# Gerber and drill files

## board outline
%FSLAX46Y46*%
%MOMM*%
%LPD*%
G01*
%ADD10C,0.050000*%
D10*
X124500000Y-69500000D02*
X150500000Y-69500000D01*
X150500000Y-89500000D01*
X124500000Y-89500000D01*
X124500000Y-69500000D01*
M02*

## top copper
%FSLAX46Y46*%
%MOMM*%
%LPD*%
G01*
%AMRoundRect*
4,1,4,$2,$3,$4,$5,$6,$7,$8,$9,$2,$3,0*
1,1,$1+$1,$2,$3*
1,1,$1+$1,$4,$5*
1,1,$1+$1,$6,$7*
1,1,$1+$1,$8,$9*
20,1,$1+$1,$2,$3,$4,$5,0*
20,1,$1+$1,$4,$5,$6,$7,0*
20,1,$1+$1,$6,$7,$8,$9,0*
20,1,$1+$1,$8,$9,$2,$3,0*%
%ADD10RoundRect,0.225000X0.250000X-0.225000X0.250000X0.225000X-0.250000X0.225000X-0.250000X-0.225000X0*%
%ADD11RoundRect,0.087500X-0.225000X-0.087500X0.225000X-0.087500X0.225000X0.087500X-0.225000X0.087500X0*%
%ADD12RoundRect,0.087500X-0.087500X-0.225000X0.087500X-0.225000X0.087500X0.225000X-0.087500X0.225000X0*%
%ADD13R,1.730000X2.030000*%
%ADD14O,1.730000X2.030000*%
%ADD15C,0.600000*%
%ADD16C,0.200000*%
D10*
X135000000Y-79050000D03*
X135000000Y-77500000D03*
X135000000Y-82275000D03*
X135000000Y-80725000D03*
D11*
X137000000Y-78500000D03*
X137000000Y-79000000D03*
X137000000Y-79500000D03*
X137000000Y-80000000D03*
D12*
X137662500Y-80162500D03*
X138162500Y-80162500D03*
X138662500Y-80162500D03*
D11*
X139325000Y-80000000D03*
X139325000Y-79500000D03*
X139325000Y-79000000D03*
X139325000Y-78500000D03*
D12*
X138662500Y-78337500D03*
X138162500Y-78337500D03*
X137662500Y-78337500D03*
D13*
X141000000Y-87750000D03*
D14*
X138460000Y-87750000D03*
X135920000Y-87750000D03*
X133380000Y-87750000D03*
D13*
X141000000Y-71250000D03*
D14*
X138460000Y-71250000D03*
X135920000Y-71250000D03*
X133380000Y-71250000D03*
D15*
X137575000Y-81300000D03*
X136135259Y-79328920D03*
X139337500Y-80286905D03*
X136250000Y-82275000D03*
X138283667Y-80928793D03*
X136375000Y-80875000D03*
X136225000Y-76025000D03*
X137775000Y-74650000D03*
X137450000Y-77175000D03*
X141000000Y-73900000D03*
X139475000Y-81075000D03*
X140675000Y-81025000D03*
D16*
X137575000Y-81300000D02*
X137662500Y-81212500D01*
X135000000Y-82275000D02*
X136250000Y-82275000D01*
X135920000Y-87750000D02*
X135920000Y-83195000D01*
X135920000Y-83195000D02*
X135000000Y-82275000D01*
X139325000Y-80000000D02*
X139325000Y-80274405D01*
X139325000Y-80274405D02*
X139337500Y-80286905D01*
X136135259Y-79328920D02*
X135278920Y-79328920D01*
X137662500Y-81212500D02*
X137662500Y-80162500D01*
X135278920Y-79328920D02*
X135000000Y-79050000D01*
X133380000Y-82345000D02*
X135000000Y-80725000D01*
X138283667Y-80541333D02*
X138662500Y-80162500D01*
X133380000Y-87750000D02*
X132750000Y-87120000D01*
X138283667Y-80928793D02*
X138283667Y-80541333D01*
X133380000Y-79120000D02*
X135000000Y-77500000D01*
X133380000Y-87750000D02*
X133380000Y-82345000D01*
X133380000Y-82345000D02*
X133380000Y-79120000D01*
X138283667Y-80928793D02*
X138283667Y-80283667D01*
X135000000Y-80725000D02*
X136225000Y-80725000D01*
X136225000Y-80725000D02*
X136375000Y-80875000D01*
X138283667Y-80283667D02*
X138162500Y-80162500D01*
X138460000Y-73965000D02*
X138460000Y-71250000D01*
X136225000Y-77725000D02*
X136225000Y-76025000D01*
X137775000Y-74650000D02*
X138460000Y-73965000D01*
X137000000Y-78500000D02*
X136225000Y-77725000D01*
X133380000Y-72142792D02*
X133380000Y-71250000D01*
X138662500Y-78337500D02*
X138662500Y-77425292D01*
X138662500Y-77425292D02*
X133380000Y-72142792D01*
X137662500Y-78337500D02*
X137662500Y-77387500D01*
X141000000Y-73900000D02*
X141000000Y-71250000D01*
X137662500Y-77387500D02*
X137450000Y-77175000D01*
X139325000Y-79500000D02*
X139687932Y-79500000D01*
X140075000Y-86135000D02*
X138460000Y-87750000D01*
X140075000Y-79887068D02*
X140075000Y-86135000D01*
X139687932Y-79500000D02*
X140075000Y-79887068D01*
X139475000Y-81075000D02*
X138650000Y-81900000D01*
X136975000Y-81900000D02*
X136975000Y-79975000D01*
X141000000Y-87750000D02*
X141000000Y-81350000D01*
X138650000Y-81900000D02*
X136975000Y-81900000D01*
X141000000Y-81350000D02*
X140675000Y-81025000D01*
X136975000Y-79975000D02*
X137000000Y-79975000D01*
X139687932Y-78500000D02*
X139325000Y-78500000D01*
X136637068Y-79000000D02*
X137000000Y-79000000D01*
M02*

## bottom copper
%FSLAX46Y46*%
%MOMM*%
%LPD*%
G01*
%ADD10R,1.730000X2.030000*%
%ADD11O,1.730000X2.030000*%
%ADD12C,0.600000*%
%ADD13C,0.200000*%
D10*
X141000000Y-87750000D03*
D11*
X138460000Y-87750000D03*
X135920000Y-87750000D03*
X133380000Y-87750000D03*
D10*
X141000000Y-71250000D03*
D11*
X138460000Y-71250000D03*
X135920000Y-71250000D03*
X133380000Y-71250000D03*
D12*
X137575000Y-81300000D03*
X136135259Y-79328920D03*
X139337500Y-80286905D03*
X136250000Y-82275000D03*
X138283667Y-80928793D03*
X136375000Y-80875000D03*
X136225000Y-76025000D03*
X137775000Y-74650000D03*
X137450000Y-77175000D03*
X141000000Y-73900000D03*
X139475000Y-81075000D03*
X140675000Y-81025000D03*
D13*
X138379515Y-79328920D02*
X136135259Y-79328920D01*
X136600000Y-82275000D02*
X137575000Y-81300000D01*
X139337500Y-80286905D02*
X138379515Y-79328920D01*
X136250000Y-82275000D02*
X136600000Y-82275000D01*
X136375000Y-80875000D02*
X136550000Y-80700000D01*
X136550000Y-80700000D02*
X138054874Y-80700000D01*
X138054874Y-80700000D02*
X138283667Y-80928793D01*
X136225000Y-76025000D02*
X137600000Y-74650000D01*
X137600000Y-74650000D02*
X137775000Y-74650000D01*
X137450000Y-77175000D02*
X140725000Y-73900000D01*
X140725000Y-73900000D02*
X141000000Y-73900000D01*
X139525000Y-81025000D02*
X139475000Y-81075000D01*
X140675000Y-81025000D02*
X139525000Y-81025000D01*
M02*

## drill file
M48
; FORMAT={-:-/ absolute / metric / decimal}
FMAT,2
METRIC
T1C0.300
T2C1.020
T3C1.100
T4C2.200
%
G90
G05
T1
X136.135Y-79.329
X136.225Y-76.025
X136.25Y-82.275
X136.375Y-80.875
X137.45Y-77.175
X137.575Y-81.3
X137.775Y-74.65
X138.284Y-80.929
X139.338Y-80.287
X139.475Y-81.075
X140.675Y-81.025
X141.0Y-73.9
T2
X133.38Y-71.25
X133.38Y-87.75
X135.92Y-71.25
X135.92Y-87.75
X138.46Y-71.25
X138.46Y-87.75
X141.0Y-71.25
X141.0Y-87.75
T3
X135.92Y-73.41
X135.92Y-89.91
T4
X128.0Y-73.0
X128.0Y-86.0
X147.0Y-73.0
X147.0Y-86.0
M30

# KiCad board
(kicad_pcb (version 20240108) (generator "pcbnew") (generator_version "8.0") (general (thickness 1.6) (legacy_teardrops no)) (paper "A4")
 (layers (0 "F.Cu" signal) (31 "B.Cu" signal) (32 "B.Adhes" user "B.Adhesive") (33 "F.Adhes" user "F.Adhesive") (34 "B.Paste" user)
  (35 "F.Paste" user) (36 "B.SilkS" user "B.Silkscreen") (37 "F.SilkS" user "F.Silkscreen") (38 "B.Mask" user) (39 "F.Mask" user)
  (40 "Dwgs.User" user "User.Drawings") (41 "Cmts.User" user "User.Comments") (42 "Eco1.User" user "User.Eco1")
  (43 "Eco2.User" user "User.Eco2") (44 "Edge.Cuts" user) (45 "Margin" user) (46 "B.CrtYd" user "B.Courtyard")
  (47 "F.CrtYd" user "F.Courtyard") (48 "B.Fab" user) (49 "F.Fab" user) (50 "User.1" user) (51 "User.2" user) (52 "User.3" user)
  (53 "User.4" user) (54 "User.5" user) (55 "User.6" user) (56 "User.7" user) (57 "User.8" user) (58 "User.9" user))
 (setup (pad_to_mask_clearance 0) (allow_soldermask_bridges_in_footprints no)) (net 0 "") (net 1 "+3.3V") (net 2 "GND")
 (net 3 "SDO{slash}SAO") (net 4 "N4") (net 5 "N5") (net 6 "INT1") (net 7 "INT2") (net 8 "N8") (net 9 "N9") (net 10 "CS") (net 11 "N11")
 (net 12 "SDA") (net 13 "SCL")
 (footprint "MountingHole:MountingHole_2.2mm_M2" (layer "F.Cu") (at 128 86)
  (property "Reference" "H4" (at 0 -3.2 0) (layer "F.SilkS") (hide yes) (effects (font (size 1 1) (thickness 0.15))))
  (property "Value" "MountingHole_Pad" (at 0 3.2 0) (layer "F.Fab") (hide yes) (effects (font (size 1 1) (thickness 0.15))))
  (pad "" np_thru_hole circle (at 0 0) (size 2.2 2.2) (drill 2.2) (layers "*.Cu" "*.Mask")))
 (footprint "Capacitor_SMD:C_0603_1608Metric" (layer "F.Cu") (at 135 78.275 90)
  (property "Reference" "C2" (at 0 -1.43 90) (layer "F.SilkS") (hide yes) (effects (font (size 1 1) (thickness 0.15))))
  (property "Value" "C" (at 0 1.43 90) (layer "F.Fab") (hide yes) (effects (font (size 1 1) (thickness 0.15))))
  (pad "1" smd roundrect (at -0.775 0 90) (size 0.9 0.95) (layers "F.Cu" "F.Paste" "F.Mask") (roundrect_rratio 0.25) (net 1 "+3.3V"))
  (pad "2" smd roundrect (at 0.775 0 90) (size 0.9 0.95) (layers "F.Cu" "F.Paste" "F.Mask") (roundrect_rratio 0.25) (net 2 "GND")))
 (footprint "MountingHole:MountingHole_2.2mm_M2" (layer "F.Cu") (at 147 86)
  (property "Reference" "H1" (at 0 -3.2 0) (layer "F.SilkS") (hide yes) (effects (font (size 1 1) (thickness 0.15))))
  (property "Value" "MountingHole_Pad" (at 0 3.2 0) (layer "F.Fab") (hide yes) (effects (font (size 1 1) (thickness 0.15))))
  (pad "" np_thru_hole circle (at 0 0) (size 2.2 2.2) (drill 2.2) (layers "*.Cu" "*.Mask")))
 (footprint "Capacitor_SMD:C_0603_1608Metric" (layer "F.Cu") (at 135 81.5 90)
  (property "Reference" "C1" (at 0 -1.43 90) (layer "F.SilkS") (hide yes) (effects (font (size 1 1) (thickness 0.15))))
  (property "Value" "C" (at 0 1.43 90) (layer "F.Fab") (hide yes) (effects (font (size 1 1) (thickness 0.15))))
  (pad "1" smd roundrect (at -0.775 0 90) (size 0.9 0.95) (layers "F.Cu" "F.Paste" "F.Mask") (roundrect_rratio 0.25) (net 1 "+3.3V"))
  (pad "2" smd roundrect (at 0.775 0 90) (size 0.9 0.95) (layers "F.Cu" "F.Paste" "F.Mask") (roundrect_rratio 0.25) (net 2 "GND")))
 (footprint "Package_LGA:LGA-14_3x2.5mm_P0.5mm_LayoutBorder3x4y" (layer "F.Cu") (at 138.1625 79.25)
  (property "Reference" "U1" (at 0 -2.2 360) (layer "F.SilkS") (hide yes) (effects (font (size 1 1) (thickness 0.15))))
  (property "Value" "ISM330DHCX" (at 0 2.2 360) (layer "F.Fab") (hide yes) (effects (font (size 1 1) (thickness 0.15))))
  (pad "1" smd roundrect (at -1.1625 -0.75) (size 0.625 0.35) (layers "F.Cu" "F.Paste" "F.Mask") (roundrect_rratio 0.25)
   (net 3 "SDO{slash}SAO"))
  (pad "2" smd roundrect (at -1.1625 -0.25) (size 0.625 0.35) (layers "F.Cu" "F.Paste" "F.Mask") (roundrect_rratio 0.25) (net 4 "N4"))
  (pad "3" smd roundrect (at -1.1625 0.25) (size 0.625 0.35) (layers "F.Cu" "F.Paste" "F.Mask") (roundrect_rratio 0.25) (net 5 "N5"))
  (pad "4" smd roundrect (at -1.1625 0.75) (size 0.625 0.35) (layers "F.Cu" "F.Paste" "F.Mask") (roundrect_rratio 0.25) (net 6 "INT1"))
  (pad "5" smd roundrect (at -0.5 0.9125) (size 0.35 0.625) (layers "F.Cu" "F.Paste" "F.Mask") (roundrect_rratio 0.25) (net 1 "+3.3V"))
  (pad "6" smd roundrect (at 0 0.9125) (size 0.35 0.625) (layers "F.Cu" "F.Paste" "F.Mask") (roundrect_rratio 0.25) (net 2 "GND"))
  (pad "7" smd roundrect (at 0.5 0.9125) (size 0.35 0.625) (layers "F.Cu" "F.Paste" "F.Mask") (roundrect_rratio 0.25) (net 2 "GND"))
  (pad "8" smd roundrect (at 1.1625 0.75) (size 0.625 0.35) (layers "F.Cu" "F.Paste" "F.Mask") (roundrect_rratio 0.25) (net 1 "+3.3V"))
  (pad "9" smd roundrect (at 1.1625 0.25) (size 0.625 0.35) (layers "F.Cu" "F.Paste" "F.Mask") (roundrect_rratio 0.25) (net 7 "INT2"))
  (pad "10" smd roundrect (at 1.1625 -0.25) (size 0.625 0.35) (layers "F.Cu" "F.Paste" "F.Mask") (roundrect_rratio 0.25) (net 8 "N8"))
  (pad "11" smd roundrect (at 1.1625 -0.75) (size 0.625 0.35) (layers "F.Cu" "F.Paste" "F.Mask") (roundrect_rratio 0.25) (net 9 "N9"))
  (pad "12" smd roundrect (at 0.5 -0.9125) (size 0.35 0.625) (layers "F.Cu" "F.Paste" "F.Mask") (roundrect_rratio 0.25) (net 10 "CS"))
  (pad "13" smd roundrect (at 0 -0.9125) (size 0.35 0.625) (layers "F.Cu" "F.Paste" "F.Mask") (roundrect_rratio 0.25) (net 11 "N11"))
  (pad "14" smd roundrect (at -0.5 -0.9125) (size 0.35 0.625) (layers "F.Cu" "F.Paste" "F.Mask") (roundrect_rratio 0.25) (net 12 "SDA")))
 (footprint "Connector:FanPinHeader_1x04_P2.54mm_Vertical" (layer "F.Cu") (at 141 87.75 180)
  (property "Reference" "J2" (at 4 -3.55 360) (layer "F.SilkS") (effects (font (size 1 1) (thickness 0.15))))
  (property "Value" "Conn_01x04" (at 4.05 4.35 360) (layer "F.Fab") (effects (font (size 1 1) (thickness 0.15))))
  (pad "" np_thru_hole circle (at 5.08 -2.16 270) (size 1.1 1.1) (drill 1.1) (layers "*.Cu" "*.Mask"))
  (pad "1" thru_hole rect (at 0 0 270) (size 2.03 1.73) (drill 1.02) (layers "*.Cu" "*.Mask") (remove_unused_layers no) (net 6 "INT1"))
  (pad "2" thru_hole oval (at 2.54 0 270) (size 2.03 1.73) (drill 1.02) (layers "*.Cu" "*.Mask") (remove_unused_layers no) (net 7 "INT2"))
  (pad "3" thru_hole oval (at 5.08 0 270) (size 2.03 1.73) (drill 1.02) (layers "*.Cu" "*.Mask") (remove_unused_layers no) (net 1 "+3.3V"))
  (pad "4" thru_hole oval (at 7.62 0 270) (size 2.03 1.73) (drill 1.02) (layers "*.Cu" "*.Mask") (remove_unused_layers no) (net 2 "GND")))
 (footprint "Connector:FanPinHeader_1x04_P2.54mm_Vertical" (layer "F.Cu") (at 141 71.25 180)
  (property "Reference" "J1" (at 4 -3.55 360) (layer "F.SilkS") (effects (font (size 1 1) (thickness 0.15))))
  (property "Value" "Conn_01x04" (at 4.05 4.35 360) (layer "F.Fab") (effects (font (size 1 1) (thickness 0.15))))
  (pad "" np_thru_hole circle (at 5.08 -2.16 270) (size 1.1 1.1) (drill 1.1) (layers "*.Cu" "*.Mask"))
  (pad "1" thru_hole rect (at 0 0 270) (size 2.03 1.73) (drill 1.02) (layers "*.Cu" "*.Mask") (remove_unused_layers no) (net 12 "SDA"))
  (pad "2" thru_hole oval (at 2.54 0 270) (size 2.03 1.73) (drill 1.02) (layers "*.Cu" "*.Mask") (remove_unused_layers no)
   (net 3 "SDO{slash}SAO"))
  (pad "3" thru_hole oval (at 5.08 0 270) (size 2.03 1.73) (drill 1.02) (layers "*.Cu" "*.Mask") (remove_unused_layers no) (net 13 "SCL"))
  (pad "4" thru_hole oval (at 7.62 0 270) (size 2.03 1.73) (drill 1.02) (layers "*.Cu" "*.Mask") (remove_unused_layers no) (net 10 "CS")))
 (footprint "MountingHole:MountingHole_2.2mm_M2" (layer "F.Cu") (at 147 73)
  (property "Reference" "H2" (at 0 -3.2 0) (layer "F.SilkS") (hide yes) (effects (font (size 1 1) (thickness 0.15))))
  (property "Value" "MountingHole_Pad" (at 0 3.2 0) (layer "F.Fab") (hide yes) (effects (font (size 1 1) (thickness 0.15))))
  (pad "" np_thru_hole circle (at 0 0) (size 2.2 2.2) (drill 2.2) (layers "*.Cu" "*.Mask")))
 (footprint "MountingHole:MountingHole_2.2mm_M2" (layer "F.Cu") (at 128 73)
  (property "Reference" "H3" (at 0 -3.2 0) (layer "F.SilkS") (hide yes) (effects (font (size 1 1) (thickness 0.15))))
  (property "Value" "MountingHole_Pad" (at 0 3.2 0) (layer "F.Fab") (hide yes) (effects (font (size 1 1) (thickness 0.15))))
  (pad "" np_thru_hole circle (at 0 0) (size 2.2 2.2) (drill 2.2) (layers "*.Cu" "*.Mask")))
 (gr_rect (start 124.5 69.5) (end 150.5 89.5) (stroke (width 0.05) (type default)) (fill none) (layer "Edge.Cuts"))
 (segment (start 137.575 81.3) (end 137.6625 81.2125) (width 0.2) (layer "F.Cu") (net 1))
 (segment (start 135 82.275) (end 136.25 82.275) (width 0.2) (layer "F.Cu") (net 1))
 (segment (start 135.92 87.75) (end 135.92 83.195) (width 0.2) (layer "F.Cu") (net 1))
 (segment (start 135.92 83.195) (end 135 82.275) (width 0.2) (layer "F.Cu") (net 1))
 (segment (start 139.325 80) (end 139.325 80.274405) (width 0.2) (layer "F.Cu") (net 1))
 (segment (start 139.325 80.274405) (end 139.3375 80.286905) (width 0.2) (layer "F.Cu") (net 1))
 (segment (start 136.135259 79.32892) (end 135.27892 79.32892) (width 0.2) (layer "F.Cu") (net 1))
 (segment (start 137.6625 81.2125) (end 137.6625 80.1625) (width 0.2) (layer "F.Cu") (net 1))
 (segment (start 135.27892 79.32892) (end 135 79.05) (width 0.2) (layer "F.Cu") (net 1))
 (via (at 137.575 81.3) (size 0.6) (drill 0.3) (layers "F.Cu" "B.Cu") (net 1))
 (via (at 136.135259 79.32892) (size 0.6) (drill 0.3) (layers "F.Cu" "B.Cu") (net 1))
 (via (at 139.3375 80.286905) (size 0.6) (drill 0.3) (layers "F.Cu" "B.Cu") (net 1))
 (via (at 136.25 82.275) (size 0.6) (drill 0.3) (layers "F.Cu" "B.Cu") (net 1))
 (segment (start 138.379515 79.32892) (end 136.135259 79.32892) (width 0.2) (layer "B.Cu") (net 1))
 (segment (start 136.6 82.275) (end 137.575 81.3) (width 0.2) (layer "B.Cu") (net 1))
 (segment (start 139.3375 80.286905) (end 138.379515 79.32892) (width 0.2) (layer "B.Cu") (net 1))
 (segment (start 136.25 82.275) (end 136.6 82.275) (width 0.2) (layer "B.Cu") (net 1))
 (segment (start 133.38 82.345) (end 135 80.725) (width 0.2) (layer "F.Cu") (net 2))
 (segment (start 138.283667 80.541333) (end 138.6625 80.1625) (width 0.2) (layer "F.Cu") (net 2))
 (segment (start 133.38 87.75) (end 132.75 87.12) (width 0.2) (layer "F.Cu") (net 2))
 (segment (start 138.283667 80.928793) (end 138.283667 80.541333) (width 0.2) (layer "F.Cu") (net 2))
 (segment (start 133.38 79.12) (end 135 77.5) (width 0.2) (layer "F.Cu") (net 2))
 (segment (start 133.38 87.75) (end 133.38 82.345) (width 0.2) (layer "F.Cu") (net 2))
 (segment (start 133.38 82.345) (end 133.38 79.12) (width 0.2) (layer "F.Cu") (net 2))
 (segment (start 138.283667 80.928793) (end 138.283667 80.283667) (width 0.2) (layer "F.Cu") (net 2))
 (segment (start 135 80.725) (end 136.225 80.725) (width 0.2) (layer "F.Cu") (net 2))
 (segment (start 136.225 80.725) (end 136.375 80.875) (width 0.2) (layer "F.Cu") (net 2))
 (segment (start 138.283667 80.283667) (end 138.1625 80.1625) (width 0.2) (layer "F.Cu") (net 2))
 (via (at 138.283667 80.928793) (size 0.6) (drill 0.3) (layers "F.Cu" "B.Cu") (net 2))
 (via (at 136.375 80.875) (size 0.6) (drill 0.3) (layers "F.Cu" "B.Cu") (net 2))
 (segment (start 136.375 80.875) (end 136.55 80.7) (width 0.2) (layer "B.Cu") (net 2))
 (segment (start 136.55 80.7) (end 138.054874 80.7) (width 0.2) (layer "B.Cu") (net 2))
 (segment (start 138.054874 80.7) (end 138.283667 80.928793) (width 0.2) (layer "B.Cu") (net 2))
 (segment (start 138.46 73.965) (end 138.46 71.25) (width 0.2) (layer "F.Cu") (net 3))
 (segment (start 136.225 77.725) (end 136.225 76.025) (width 0.2) (layer "F.Cu") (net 3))
 (segment (start 137.775 74.65) (end 138.46 73.965) (width 0.2) (layer "F.Cu") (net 3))
 (segment (start 137 78.5) (end 136.225 77.725) (width 0.2) (layer "F.Cu") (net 3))
 (via (at 136.225 76.025) (size 0.6) (drill 0.3) (layers "F.Cu" "B.Cu") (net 3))
 (via (at 137.775 74.65) (size 0.6) (drill 0.3) (layers "F.Cu" "B.Cu") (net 3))
 (segment (start 136.225 76.025) (end 137.6 74.65) (width 0.2) (layer "B.Cu") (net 3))
 (segment (start 137.6 74.65) (end 137.775 74.65) (width 0.2) (layer "B.Cu") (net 3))
 (segment (start 133.38 72.142792) (end 133.38 71.25) (width 0.2) (layer "F.Cu") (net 10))
 (segment (start 138.6625 78.3375) (end 138.6625 77.425292) (width 0.2) (layer "F.Cu") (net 10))
 (segment (start 138.6625 77.425292) (end 133.38 72.142792) (width 0.2) (layer "F.Cu") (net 10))
 (segment (start 137.6625 78.3375) (end 137.6625 77.3875) (width 0.2) (layer "F.Cu") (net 12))
 (segment (start 141 73.9) (end 141 71.25) (width 0.2) (layer "F.Cu") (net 12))
 (segment (start 137.6625 77.3875) (end 137.45 77.175) (width 0.2) (layer "F.Cu") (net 12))
 (via (at 137.45 77.175) (size 0.6) (drill 0.3) (layers "F.Cu" "B.Cu") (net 12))
 (via (at 141 73.9) (size 0.6) (drill 0.3) (layers "F.Cu" "B.Cu") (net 12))
 (segment (start 137.45 77.175) (end 140.725 73.9) (width 0.2) (layer "B.Cu") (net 12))
 (segment (start 140.725 73.9) (end 141 73.9) (width 0.2) (layer "B.Cu") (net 12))
 (segment (start 139.325 79.5) (end 139.687932 79.5) (width 0.2) (layer "F.Cu") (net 7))
 (segment (start 140.075 86.135) (end 138.46 87.75) (width 0.2) (layer "F.Cu") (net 7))
 (segment (start 140.075 79.887068) (end 140.075 86.135) (width 0.2) (layer "F.Cu") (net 7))
 (segment (start 139.687932 79.5) (end 140.075 79.887068) (width 0.2) (layer "F.Cu") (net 7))
 (segment (start 139.475 81.075) (end 138.65 81.9) (width 0.2) (layer "F.Cu") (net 6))
 (segment (start 136.975 81.9) (end 136.975 79.975) (width 0.2) (layer "F.Cu") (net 6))
 (segment (start 141 87.75) (end 141 81.35) (width 0.2) (layer "F.Cu") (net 6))
 (segment (start 138.65 81.9) (end 136.975 81.9) (width 0.2) (layer "F.Cu") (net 6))
 (segment (start 141 81.35) (end 140.675 81.025) (width 0.2) (layer "F.Cu") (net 6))
 (segment (start 136.975 79.975) (end 137 79.975) (width 0.2) (layer "F.Cu") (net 6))
 (via (at 139.475 81.075) (size 0.6) (drill 0.3) (layers "F.Cu" "B.Cu") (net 6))
 (via (at 140.675 81.025) (size 0.6) (drill 0.3) (layers "F.Cu" "B.Cu") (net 6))
 (segment (start 139.525 81.025) (end 139.475 81.075) (width 0.2) (layer "B.Cu") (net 6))
 (segment (start 140.675 81.025) (end 139.525 81.025) (width 0.2) (layer "B.Cu") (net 6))
 (segment (start 139.687932 78.5) (end 139.325 78.5) (width 0.2) (layer "F.Cu") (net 9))
 (segment (start 136.637068 79) (end 137 79) (width 0.2) (layer "F.Cu") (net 4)))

